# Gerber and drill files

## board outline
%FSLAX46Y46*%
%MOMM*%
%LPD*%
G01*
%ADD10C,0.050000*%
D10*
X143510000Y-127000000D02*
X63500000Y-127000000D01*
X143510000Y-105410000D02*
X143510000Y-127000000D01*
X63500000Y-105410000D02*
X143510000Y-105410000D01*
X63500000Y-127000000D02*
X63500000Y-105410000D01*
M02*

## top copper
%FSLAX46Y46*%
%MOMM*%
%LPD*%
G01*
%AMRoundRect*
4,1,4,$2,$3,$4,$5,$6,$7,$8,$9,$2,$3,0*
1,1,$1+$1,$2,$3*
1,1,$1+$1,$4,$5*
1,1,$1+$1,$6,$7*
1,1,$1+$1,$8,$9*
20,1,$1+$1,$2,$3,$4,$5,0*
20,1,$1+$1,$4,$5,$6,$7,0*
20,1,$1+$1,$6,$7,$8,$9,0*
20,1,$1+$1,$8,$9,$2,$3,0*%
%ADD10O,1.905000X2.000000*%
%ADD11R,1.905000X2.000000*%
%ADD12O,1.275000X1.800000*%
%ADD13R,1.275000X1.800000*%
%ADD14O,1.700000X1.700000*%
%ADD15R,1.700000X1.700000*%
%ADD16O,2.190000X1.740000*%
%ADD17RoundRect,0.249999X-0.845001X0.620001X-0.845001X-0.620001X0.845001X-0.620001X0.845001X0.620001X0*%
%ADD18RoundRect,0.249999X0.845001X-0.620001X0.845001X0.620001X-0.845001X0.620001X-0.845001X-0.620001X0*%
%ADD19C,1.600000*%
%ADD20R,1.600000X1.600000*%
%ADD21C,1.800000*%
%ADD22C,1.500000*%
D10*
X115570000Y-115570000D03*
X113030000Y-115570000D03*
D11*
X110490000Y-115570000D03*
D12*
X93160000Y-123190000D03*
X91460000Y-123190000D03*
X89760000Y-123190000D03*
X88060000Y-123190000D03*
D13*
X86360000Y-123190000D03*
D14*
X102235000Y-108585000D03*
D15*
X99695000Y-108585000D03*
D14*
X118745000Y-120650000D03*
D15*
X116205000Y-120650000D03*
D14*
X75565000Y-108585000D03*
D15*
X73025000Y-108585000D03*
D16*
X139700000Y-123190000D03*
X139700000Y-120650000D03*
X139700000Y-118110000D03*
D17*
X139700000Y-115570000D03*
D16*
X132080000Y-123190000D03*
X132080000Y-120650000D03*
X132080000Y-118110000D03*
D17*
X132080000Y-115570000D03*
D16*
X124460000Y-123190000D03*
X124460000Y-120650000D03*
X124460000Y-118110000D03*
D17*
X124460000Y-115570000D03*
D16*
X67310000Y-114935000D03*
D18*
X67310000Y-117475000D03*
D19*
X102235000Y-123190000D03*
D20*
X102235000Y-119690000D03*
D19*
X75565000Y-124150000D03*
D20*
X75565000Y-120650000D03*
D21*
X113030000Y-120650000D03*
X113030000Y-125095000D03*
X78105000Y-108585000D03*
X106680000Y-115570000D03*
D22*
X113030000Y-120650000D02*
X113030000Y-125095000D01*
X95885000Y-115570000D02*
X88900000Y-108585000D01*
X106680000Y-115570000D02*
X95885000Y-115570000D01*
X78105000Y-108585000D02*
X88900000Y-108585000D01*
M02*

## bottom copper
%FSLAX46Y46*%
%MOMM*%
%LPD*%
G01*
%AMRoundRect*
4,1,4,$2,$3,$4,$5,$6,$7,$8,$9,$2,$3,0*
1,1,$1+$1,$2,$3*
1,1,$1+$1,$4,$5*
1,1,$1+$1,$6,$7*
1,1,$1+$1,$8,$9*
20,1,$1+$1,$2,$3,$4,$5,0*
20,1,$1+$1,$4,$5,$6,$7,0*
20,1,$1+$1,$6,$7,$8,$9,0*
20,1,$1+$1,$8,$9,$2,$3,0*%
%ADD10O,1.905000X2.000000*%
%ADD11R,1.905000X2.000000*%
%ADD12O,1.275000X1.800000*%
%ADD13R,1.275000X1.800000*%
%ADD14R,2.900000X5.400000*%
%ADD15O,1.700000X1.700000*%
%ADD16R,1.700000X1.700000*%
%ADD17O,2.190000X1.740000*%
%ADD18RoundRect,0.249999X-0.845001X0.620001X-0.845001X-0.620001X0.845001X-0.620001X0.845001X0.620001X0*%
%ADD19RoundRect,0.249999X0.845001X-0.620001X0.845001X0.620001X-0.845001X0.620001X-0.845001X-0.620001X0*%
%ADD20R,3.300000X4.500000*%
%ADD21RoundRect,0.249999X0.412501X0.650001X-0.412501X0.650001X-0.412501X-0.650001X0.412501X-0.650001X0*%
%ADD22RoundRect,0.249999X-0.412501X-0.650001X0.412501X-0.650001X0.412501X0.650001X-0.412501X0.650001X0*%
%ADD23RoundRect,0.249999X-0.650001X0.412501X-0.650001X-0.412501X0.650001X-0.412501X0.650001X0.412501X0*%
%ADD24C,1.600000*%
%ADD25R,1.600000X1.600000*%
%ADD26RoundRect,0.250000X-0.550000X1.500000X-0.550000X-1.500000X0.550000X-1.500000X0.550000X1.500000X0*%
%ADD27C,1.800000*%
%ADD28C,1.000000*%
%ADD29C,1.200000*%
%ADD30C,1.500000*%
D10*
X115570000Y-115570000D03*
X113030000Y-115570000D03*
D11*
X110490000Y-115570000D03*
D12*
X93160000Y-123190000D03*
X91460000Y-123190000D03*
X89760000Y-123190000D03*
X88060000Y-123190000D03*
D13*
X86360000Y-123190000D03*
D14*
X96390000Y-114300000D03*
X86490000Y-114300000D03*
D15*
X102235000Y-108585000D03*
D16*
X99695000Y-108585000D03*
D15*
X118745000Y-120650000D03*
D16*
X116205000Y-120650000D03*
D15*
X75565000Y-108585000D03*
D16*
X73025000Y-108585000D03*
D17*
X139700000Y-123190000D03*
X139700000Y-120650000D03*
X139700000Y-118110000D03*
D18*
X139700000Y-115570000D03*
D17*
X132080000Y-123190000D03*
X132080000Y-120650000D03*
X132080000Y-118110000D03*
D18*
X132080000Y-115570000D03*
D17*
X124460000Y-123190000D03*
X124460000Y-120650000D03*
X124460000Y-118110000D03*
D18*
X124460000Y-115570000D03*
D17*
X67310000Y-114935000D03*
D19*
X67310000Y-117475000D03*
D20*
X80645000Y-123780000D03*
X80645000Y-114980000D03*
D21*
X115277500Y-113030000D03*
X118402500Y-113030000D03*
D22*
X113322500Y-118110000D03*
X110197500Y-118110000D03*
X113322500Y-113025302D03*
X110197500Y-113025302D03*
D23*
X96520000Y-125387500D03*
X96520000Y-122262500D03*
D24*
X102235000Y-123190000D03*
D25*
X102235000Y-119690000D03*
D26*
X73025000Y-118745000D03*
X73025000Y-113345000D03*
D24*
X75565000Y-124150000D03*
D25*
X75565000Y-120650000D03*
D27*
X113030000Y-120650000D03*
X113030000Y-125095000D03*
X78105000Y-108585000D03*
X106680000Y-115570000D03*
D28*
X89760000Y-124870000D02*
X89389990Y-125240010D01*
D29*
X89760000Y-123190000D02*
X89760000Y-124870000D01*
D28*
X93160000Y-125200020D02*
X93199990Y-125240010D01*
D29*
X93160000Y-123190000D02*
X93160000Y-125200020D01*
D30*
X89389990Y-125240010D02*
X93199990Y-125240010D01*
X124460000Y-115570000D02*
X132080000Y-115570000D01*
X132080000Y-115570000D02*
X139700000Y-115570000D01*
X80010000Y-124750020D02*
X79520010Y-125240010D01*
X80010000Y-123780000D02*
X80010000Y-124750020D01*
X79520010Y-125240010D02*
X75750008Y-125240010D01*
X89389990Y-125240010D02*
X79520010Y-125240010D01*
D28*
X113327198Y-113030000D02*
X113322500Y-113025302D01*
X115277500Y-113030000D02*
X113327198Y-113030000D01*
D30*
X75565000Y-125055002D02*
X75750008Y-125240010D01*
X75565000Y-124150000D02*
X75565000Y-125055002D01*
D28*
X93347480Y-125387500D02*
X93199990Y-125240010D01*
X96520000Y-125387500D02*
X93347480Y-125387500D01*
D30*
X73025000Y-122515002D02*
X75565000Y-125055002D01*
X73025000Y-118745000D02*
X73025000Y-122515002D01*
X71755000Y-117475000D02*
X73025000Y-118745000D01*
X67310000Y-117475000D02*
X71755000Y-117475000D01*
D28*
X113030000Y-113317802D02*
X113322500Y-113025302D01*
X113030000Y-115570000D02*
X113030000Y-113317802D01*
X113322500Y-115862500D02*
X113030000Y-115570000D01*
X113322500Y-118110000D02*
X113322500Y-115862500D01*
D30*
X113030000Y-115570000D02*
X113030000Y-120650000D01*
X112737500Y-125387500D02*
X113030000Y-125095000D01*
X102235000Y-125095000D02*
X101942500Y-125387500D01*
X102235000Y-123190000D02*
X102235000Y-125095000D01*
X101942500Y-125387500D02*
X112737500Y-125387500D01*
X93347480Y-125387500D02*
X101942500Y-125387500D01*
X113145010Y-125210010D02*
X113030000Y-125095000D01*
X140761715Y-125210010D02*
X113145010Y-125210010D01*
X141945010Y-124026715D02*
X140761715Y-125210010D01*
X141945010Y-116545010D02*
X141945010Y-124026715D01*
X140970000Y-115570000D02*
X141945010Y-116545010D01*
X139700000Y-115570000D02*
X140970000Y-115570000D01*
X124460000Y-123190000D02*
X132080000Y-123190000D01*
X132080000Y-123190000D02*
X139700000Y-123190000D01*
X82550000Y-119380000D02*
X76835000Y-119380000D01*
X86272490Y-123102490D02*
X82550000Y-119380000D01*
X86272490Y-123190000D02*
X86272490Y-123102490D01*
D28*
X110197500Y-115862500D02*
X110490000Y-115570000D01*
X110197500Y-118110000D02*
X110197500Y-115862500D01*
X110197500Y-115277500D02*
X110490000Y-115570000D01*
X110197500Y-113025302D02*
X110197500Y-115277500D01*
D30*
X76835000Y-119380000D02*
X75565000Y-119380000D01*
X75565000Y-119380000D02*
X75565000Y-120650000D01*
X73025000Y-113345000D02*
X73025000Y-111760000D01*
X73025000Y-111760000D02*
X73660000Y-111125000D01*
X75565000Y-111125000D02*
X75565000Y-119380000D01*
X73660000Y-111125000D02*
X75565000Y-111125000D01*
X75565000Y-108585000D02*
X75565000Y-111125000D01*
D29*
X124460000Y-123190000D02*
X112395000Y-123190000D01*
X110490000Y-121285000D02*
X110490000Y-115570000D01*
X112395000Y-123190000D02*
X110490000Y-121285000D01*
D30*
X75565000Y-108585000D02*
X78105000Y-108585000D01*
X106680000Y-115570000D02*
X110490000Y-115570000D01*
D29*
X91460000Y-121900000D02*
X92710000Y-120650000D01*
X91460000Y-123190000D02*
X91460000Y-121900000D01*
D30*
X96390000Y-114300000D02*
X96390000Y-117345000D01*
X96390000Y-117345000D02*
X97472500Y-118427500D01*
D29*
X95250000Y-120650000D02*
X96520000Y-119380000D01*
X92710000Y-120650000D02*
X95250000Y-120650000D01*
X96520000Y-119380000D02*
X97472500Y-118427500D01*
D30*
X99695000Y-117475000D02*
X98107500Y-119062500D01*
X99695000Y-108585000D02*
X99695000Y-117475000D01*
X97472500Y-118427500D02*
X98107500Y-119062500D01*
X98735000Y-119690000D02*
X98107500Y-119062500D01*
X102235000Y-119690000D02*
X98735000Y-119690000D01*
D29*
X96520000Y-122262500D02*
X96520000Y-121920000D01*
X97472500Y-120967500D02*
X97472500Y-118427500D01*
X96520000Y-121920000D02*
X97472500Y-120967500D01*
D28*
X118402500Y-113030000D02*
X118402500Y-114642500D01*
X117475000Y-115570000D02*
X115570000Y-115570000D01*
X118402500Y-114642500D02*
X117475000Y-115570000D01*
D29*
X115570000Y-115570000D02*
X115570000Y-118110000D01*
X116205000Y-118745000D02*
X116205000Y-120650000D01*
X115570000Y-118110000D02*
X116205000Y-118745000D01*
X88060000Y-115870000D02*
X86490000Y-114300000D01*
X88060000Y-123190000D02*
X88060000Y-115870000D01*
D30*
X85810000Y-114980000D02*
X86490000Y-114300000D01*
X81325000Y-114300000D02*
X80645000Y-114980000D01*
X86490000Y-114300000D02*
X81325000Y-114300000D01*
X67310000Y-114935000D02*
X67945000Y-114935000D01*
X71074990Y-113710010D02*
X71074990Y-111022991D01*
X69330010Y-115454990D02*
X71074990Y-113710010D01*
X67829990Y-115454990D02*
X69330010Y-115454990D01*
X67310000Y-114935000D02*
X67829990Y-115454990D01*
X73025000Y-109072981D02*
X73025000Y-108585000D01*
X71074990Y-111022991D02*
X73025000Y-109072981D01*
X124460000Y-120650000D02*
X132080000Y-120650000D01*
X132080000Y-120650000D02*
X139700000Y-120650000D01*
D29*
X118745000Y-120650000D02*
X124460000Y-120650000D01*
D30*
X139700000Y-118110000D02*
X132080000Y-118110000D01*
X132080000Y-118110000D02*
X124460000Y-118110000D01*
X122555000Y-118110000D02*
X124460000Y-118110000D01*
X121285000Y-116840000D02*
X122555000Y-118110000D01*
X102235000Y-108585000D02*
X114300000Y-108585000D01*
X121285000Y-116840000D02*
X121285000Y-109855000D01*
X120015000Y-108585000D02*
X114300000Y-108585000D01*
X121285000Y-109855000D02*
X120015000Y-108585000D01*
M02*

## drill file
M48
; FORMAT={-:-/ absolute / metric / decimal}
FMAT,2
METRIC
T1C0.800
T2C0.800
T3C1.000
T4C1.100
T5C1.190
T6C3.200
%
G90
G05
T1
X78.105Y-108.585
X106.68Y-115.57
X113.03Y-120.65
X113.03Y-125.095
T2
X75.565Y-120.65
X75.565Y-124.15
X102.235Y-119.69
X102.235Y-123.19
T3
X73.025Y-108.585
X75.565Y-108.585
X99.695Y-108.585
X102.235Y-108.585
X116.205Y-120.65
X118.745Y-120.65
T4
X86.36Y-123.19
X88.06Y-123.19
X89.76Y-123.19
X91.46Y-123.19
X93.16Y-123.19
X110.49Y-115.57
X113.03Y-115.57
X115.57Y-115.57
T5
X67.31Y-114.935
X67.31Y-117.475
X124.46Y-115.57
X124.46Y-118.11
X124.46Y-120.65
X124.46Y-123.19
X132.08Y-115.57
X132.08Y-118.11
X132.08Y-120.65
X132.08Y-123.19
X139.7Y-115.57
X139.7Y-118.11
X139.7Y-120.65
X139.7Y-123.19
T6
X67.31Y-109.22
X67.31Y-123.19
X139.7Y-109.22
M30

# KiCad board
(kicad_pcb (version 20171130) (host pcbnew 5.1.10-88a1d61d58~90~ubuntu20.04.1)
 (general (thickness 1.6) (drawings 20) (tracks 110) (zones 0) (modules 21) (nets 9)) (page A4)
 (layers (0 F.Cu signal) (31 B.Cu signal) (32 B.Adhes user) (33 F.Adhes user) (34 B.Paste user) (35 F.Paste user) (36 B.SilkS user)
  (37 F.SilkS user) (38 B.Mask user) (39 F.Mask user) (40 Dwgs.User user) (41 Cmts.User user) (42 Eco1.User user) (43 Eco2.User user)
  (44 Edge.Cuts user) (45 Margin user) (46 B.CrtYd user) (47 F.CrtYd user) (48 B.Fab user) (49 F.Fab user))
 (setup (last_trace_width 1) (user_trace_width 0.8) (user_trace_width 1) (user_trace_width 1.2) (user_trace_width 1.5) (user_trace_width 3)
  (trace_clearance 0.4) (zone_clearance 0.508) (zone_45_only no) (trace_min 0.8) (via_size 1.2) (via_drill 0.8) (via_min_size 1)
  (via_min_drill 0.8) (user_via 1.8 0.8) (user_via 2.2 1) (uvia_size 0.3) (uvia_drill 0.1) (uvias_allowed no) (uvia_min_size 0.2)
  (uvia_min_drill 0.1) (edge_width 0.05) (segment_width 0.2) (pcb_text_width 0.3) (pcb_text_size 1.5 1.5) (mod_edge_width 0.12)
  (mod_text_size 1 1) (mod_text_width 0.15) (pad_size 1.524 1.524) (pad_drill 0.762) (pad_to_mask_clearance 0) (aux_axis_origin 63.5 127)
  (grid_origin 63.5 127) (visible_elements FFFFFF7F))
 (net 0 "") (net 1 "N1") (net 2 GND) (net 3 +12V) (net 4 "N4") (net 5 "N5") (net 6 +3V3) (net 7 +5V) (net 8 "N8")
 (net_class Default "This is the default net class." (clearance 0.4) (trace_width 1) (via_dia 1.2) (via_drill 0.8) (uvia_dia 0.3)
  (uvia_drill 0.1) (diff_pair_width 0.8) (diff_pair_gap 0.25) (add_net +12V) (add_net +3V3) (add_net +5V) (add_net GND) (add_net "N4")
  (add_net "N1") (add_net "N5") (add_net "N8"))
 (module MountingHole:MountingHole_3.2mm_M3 (layer F.Cu) (at 139.7 109.22)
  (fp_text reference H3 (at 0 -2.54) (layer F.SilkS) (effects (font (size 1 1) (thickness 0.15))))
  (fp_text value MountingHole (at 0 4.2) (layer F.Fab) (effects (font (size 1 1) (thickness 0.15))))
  (pad 1 np_thru_hole circle (at 0 0) (size 3.2 3.2) (drill 3.2) (layers *.Cu *.Mask)))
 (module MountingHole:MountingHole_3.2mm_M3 (layer F.Cu) (at 67.31 123.19)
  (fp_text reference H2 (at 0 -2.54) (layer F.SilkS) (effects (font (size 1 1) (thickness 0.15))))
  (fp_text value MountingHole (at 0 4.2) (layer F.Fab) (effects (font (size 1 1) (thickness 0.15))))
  (pad 1 np_thru_hole circle (at 0 0) (size 3.2 3.2) (drill 3.2) (layers *.Cu *.Mask)))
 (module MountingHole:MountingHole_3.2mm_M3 (layer F.Cu) (at 67.31 109.22)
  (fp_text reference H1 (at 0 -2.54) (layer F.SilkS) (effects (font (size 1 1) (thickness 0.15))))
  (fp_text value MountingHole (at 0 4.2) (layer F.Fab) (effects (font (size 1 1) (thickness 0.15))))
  (pad 1 np_thru_hole circle (at 0 0) (size 3.2 3.2) (drill 3.2) (layers *.Cu *.Mask)))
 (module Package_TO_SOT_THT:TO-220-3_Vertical (layer F.Cu) (at 110.49 115.57)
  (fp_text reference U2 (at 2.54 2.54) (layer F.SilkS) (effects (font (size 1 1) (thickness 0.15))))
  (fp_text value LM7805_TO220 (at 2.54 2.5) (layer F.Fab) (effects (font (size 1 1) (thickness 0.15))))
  (pad 3 thru_hole oval (at 5.08 0) (size 1.905 2) (drill 1.1) (layers *.Cu *.Mask) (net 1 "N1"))
  (pad 2 thru_hole oval (at 2.54 0) (size 1.905 2) (drill 1.1) (layers *.Cu *.Mask) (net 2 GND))
  (pad 1 thru_hole rect (at 0 0) (size 1.905 2) (drill 1.1) (layers *.Cu *.Mask) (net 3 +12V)))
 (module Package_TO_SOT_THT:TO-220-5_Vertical (layer F.Cu) (at 86.36 123.19)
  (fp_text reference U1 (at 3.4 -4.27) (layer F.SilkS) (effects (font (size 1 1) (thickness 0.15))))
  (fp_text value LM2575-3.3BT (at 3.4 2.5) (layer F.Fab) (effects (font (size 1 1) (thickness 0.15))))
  (pad 5 thru_hole oval (at 6.8 0) (size 1.275 1.8) (drill 1.1) (layers *.Cu *.Mask) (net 2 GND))
  (pad 4 thru_hole oval (at 5.1 0) (size 1.275 1.8) (drill 1.1) (layers *.Cu *.Mask) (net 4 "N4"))
  (pad 3 thru_hole oval (at 3.4 0) (size 1.275 1.8) (drill 1.1) (layers *.Cu *.Mask) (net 2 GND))
  (pad 2 thru_hole oval (at 1.7 0) (size 1.275 1.8) (drill 1.1) (layers *.Cu *.Mask) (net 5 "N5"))
  (pad 1 thru_hole rect (at 0 0) (size 1.275 1.8) (drill 1.1) (layers *.Cu *.Mask) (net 3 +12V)))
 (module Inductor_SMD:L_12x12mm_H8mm (layer B.Cu) (at 91.44 114.3)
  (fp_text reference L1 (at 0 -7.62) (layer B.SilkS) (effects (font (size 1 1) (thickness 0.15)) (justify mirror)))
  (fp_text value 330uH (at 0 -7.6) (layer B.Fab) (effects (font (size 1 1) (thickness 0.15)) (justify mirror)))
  (pad 2 smd rect (at 4.95 0) (size 2.9 5.4) (layers B.Cu B.Paste B.Mask) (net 4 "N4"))
  (pad 1 smd rect (at -4.95 0) (size 2.9 5.4) (layers B.Cu B.Paste B.Mask) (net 5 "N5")))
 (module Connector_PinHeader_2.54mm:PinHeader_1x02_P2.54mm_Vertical (layer F.Cu) (at 99.695 108.585 90)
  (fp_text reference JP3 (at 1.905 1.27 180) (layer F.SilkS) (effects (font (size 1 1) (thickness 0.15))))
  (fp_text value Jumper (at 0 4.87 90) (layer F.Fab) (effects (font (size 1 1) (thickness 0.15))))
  (pad 2 thru_hole oval (at 0 2.54 90) (size 1.7 1.7) (drill 1) (layers *.Cu *.Mask) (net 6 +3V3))
  (pad 1 thru_hole rect (at 0 0 90) (size 1.7 1.7) (drill 1) (layers *.Cu *.Mask) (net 4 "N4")))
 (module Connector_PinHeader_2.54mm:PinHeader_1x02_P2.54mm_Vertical (layer F.Cu) (at 116.205 120.65 90)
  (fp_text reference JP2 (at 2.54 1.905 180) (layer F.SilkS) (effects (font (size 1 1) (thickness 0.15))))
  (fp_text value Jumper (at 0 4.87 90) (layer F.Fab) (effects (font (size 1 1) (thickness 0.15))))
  (pad 2 thru_hole oval (at 0 2.54 90) (size 1.7 1.7) (drill 1) (layers *.Cu *.Mask) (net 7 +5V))
  (pad 1 thru_hole rect (at 0 0 90) (size 1.7 1.7) (drill 1) (layers *.Cu *.Mask) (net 1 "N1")))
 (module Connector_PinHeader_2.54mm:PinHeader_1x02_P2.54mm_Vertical (layer F.Cu) (at 73.025 108.585 90)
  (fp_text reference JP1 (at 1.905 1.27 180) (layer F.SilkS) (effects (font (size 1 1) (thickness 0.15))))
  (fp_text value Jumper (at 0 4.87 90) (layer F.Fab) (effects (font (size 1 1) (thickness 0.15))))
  (pad 2 thru_hole oval (at 0 2.54 90) (size 1.7 1.7) (drill 1) (layers *.Cu *.Mask) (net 3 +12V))
  (pad 1 thru_hole rect (at 0 0 90) (size 1.7 1.7) (drill 1) (layers *.Cu *.Mask) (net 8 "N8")))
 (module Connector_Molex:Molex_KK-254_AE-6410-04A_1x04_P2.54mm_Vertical (layer F.Cu) (at 139.7 115.57 270)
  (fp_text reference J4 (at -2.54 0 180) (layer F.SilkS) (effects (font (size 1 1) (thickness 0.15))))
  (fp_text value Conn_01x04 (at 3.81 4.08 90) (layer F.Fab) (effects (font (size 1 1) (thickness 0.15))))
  (pad 4 thru_hole oval (at 7.62 0 270) (size 1.74 2.19) (drill 1.19) (layers *.Cu *.Mask) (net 3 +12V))
  (pad 3 thru_hole oval (at 5.08 0 270) (size 1.74 2.19) (drill 1.19) (layers *.Cu *.Mask) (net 7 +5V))
  (pad 2 thru_hole oval (at 2.54 0 270) (size 1.74 2.19) (drill 1.19) (layers *.Cu *.Mask) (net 6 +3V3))
  (pad 1 thru_hole roundrect (at 0 0 270) (size 1.74 2.19) (drill 1.19) (layers *.Cu *.Mask) (roundrect_rratio 0.1436775862068966)
   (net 2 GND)))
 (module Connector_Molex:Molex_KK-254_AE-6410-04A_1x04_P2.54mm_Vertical (layer F.Cu) (at 132.08 115.57 270)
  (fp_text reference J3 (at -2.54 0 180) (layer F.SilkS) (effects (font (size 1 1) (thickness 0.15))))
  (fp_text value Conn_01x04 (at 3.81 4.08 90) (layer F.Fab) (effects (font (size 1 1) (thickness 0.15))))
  (pad 4 thru_hole oval (at 7.62 0 270) (size 1.74 2.19) (drill 1.19) (layers *.Cu *.Mask) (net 3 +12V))
  (pad 3 thru_hole oval (at 5.08 0 270) (size 1.74 2.19) (drill 1.19) (layers *.Cu *.Mask) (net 7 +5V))
  (pad 2 thru_hole oval (at 2.54 0 270) (size 1.74 2.19) (drill 1.19) (layers *.Cu *.Mask) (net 6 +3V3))
  (pad 1 thru_hole roundrect (at 0 0 270) (size 1.74 2.19) (drill 1.19) (layers *.Cu *.Mask) (roundrect_rratio 0.1436775862068966)
   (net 2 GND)))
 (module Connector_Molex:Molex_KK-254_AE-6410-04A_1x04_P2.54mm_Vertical (layer F.Cu) (at 124.46 115.57 270)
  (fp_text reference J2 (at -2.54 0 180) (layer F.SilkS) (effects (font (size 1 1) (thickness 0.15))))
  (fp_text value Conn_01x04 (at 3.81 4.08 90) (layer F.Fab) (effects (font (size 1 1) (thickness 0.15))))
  (pad 4 thru_hole oval (at 7.62 0 270) (size 1.74 2.19) (drill 1.19) (layers *.Cu *.Mask) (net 3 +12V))
  (pad 3 thru_hole oval (at 5.08 0 270) (size 1.74 2.19) (drill 1.19) (layers *.Cu *.Mask) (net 7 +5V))
  (pad 2 thru_hole oval (at 2.54 0 270) (size 1.74 2.19) (drill 1.19) (layers *.Cu *.Mask) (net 6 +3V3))
  (pad 1 thru_hole roundrect (at 0 0 270) (size 1.74 2.19) (drill 1.19) (layers *.Cu *.Mask) (roundrect_rratio 0.1436775862068966)
   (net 2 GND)))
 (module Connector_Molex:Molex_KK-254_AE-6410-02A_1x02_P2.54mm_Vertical (layer F.Cu) (at 67.31 117.475 90)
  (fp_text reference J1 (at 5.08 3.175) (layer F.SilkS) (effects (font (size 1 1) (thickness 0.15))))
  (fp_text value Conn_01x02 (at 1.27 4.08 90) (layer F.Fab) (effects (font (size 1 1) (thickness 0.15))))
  (pad 2 thru_hole oval (at 2.54 0 90) (size 1.74 2.19) (drill 1.19) (layers *.Cu *.Mask) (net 8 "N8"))
  (pad 1 thru_hole roundrect (at 0 0 90) (size 1.74 2.19) (drill 1.19) (layers *.Cu *.Mask) (roundrect_rratio 0.1436775862068966)
   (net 2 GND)))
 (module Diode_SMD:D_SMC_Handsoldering (layer B.Cu) (at 80.645 119.38 270)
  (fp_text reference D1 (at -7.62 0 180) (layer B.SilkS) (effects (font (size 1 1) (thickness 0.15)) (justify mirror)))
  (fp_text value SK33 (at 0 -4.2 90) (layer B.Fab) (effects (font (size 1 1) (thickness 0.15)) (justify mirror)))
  (pad 2 smd rect (at 4.4 0 180) (size 3.3 4.5) (layers B.Cu B.Paste B.Mask) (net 2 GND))
  (pad 1 smd rect (at -4.4 0 180) (size 3.3 4.5) (layers B.Cu B.Paste B.Mask) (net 5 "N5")))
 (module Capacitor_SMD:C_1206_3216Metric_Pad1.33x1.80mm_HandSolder (layer B.Cu) (at 116.84 113.03 180)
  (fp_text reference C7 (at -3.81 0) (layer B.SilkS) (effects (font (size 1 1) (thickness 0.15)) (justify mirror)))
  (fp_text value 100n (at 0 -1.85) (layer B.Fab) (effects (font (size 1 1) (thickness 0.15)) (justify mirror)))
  (pad 2 smd roundrect (at 1.5625 0 180) (size 1.325 1.8) (layers B.Cu B.Paste B.Mask) (roundrect_rratio 0.1886784905660377) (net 2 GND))
  (pad 1 smd roundrect (at -1.5625 0 180) (size 1.325 1.8) (layers B.Cu B.Paste B.Mask) (roundrect_rratio 0.1886784905660377) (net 1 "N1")))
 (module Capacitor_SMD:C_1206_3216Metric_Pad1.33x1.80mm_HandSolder (layer B.Cu) (at 111.76 118.11)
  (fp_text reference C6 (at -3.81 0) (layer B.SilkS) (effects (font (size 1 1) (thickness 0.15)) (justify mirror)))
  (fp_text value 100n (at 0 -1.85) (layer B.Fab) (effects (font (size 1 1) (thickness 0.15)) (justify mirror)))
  (pad 2 smd roundrect (at 1.5625 0) (size 1.325 1.8) (layers B.Cu B.Paste B.Mask) (roundrect_rratio 0.1886784905660377) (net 2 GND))
  (pad 1 smd roundrect (at -1.5625 0) (size 1.325 1.8) (layers B.Cu B.Paste B.Mask) (roundrect_rratio 0.1886784905660377) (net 3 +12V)))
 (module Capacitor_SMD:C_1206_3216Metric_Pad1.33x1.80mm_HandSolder (layer B.Cu) (at 111.76 113.025302)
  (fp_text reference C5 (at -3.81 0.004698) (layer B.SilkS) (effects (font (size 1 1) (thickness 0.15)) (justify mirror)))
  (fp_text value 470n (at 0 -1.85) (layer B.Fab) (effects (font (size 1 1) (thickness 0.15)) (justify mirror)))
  (pad 2 smd roundrect (at 1.5625 0) (size 1.325 1.8) (layers B.Cu B.Paste B.Mask) (roundrect_rratio 0.1886784905660377) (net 2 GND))
  (pad 1 smd roundrect (at -1.5625 0) (size 1.325 1.8) (layers B.Cu B.Paste B.Mask) (roundrect_rratio 0.1886784905660377) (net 3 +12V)))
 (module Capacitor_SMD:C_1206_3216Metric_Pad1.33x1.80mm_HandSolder (layer B.Cu) (at 96.52 123.825 270)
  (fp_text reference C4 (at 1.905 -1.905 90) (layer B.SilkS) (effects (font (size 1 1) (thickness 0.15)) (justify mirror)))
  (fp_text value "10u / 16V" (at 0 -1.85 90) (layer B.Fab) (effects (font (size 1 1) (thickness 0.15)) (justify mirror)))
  (pad 2 smd roundrect (at 1.5625 0 270) (size 1.325 1.8) (layers B.Cu B.Paste B.Mask) (roundrect_rratio 0.1886784905660377) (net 2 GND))
  (pad 1 smd roundrect (at -1.5625 0 270) (size 1.325 1.8) (layers B.Cu B.Paste B.Mask) (roundrect_rratio 0.1886784905660377) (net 4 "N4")))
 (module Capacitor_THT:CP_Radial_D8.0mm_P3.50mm (layer F.Cu) (at 102.235 119.69 270)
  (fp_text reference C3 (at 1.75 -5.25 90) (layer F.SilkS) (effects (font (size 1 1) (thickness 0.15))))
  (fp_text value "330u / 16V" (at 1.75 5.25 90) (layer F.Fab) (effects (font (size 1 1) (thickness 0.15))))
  (pad 2 thru_hole circle (at 3.5 0 270) (size 1.6 1.6) (drill 0.8) (layers *.Cu *.Mask) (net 2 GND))
  (pad 1 thru_hole rect (at 0 0 270) (size 1.6 1.6) (drill 0.8) (layers *.Cu *.Mask) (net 4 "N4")))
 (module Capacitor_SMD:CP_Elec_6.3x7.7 (layer B.Cu) (at 73.025 116.045 270)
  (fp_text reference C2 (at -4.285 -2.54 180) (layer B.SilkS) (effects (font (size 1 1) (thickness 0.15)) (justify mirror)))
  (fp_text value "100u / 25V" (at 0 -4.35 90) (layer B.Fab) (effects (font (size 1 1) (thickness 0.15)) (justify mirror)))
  (pad 2 smd roundrect (at 2.7 0 270) (size 3.5 1.6) (layers B.Cu B.Paste B.Mask) (roundrect_rratio 0.15625) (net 2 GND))
  (pad 1 smd roundrect (at -2.7 0 270) (size 3.5 1.6) (layers B.Cu B.Paste B.Mask) (roundrect_rratio 0.15625) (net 3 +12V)))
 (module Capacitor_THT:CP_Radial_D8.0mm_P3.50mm (layer F.Cu) (at 75.565 120.65 270)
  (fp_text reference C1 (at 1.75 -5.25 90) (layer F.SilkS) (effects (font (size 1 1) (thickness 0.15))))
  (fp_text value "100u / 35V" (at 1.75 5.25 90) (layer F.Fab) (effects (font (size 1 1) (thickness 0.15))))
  (pad 2 thru_hole circle (at 3.5 0 270) (size 1.6 1.6) (drill 0.8) (layers *.Cu *.Mask) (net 2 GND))
  (pad 1 thru_hole rect (at 0 0 270) (size 1.6 1.6) (drill 0.8) (layers *.Cu *.Mask) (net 3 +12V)))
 (gr_line (start 143.51 127) (end 63.5 127) (layer Edge.Cuts) (width 0.05))
 (gr_line (start 143.51 105.41) (end 143.51 127) (layer Edge.Cuts) (width 0.05))
 (gr_line (start 63.5 105.41) (end 143.51 105.41) (layer Edge.Cuts) (width 0.05))
 (gr_line (start 63.5 127) (end 63.5 105.41) (layer Edge.Cuts) (width 0.05))
 (segment (start 89.76 124.87) (end 89.38999 125.24001) (width 1) (layer B.Cu) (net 2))
 (segment (start 89.76 123.19) (end 89.76 124.87) (width 1.2) (layer B.Cu) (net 2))
 (segment (start 93.16 125.20002) (end 93.19999 125.24001) (width 1) (layer B.Cu) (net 2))
 (segment (start 93.16 123.19) (end 93.16 125.20002) (width 1.2) (layer B.Cu) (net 2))
 (segment (start 89.38999 125.24001) (end 93.19999 125.24001) (width 1.5) (layer B.Cu) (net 2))
 (segment (start 124.46 115.57) (end 132.08 115.57) (width 1.5) (layer B.Cu) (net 2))
 (segment (start 132.08 115.57) (end 139.7 115.57) (width 1.5) (layer B.Cu) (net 2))
 (segment (start 80.01 124.75002) (end 79.52001 125.24001) (width 1.5) (layer B.Cu) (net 2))
 (segment (start 80.01 123.78) (end 80.01 124.75002) (width 1.5) (layer B.Cu) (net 2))
 (segment (start 79.52001 125.24001) (end 75.750008 125.24001) (width 1.5) (layer B.Cu) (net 2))
 (segment (start 89.38999 125.24001) (end 79.52001 125.24001) (width 1.5) (layer B.Cu) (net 2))
 (segment (start 113.327198 113.03) (end 113.3225 113.025302) (width 1) (layer B.Cu) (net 2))
 (segment (start 115.2775 113.03) (end 113.327198 113.03) (width 1) (layer B.Cu) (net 2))
 (segment (start 75.565 125.055002) (end 75.750008 125.24001) (width 1.5) (layer B.Cu) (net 2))
 (segment (start 75.565 124.15) (end 75.565 125.055002) (width 1.5) (layer B.Cu) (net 2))
 (segment (start 93.34748 125.3875) (end 93.19999 125.24001) (width 1) (layer B.Cu) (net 2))
 (segment (start 96.52 125.3875) (end 93.34748 125.3875) (width 1) (layer B.Cu) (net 2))
 (segment (start 73.025 122.515002) (end 75.565 125.055002) (width 1.5) (layer B.Cu) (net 2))
 (segment (start 73.025 118.745) (end 73.025 122.515002) (width 1.5) (layer B.Cu) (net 2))
 (segment (start 71.755 117.475) (end 73.025 118.745) (width 1.5) (layer B.Cu) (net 2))
 (segment (start 67.31 117.475) (end 71.755 117.475) (width 1.5) (layer B.Cu) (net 2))
 (segment (start 113.03 113.317802) (end 113.3225 113.025302) (width 1) (layer B.Cu) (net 2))
 (segment (start 113.03 115.57) (end 113.03 113.317802) (width 1) (layer B.Cu) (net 2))
 (segment (start 113.3225 115.8625) (end 113.03 115.57) (width 1) (layer B.Cu) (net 2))
 (segment (start 113.3225 118.11) (end 113.3225 115.8625) (width 1) (layer B.Cu) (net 2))
 (via (at 113.03 120.65) (size 1.8) (drill 0.8) (layers F.Cu B.Cu) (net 2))
 (segment (start 113.03 115.57) (end 113.03 120.65) (width 1.5) (layer B.Cu) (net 2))
 (via (at 113.03 125.095) (size 1.8) (drill 0.8) (layers F.Cu B.Cu) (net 2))
 (segment (start 113.03 120.65) (end 113.03 125.095) (width 1.5) (layer F.Cu) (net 2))
 (segment (start 112.7375 125.3875) (end 113.03 125.095) (width 1.5) (layer B.Cu) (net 2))
 (segment (start 102.235 125.095) (end 101.9425 125.3875) (width 1.5) (layer B.Cu) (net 2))
 (segment (start 102.235 123.19) (end 102.235 125.095) (width 1.5) (layer B.Cu) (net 2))
 (segment (start 101.9425 125.3875) (end 112.7375 125.3875) (width 1.5) (layer B.Cu) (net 2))
 (segment (start 93.34748 125.3875) (end 101.9425 125.3875) (width 1.5) (layer B.Cu) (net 2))
 (segment (start 113.14501 125.21001) (end 113.03 125.095) (width 1.5) (layer B.Cu) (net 2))
 (segment (start 140.761715 125.21001) (end 113.14501 125.21001) (width 1.5) (layer B.Cu) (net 2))
 (segment (start 141.94501 124.026715) (end 140.761715 125.21001) (width 1.5) (layer B.Cu) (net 2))
 (segment (start 141.94501 116.54501) (end 141.94501 124.026715) (width 1.5) (layer B.Cu) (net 2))
 (segment (start 140.97 115.57) (end 141.94501 116.54501) (width 1.5) (layer B.Cu) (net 2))
 (segment (start 139.7 115.57) (end 140.97 115.57) (width 1.5) (layer B.Cu) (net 2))
 (segment (start 124.46 123.19) (end 132.08 123.19) (width 1.5) (layer B.Cu) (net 3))
 (segment (start 132.08 123.19) (end 139.7 123.19) (width 1.5) (layer B.Cu) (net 3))
 (segment (start 82.55 119.38) (end 76.835 119.38) (width 1.5) (layer B.Cu) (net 3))
 (segment (start 86.27249 123.10249) (end 82.55 119.38) (width 1.5) (layer B.Cu) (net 3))
 (segment (start 86.27249 123.19) (end 86.27249 123.10249) (width 1.5) (layer B.Cu) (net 3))
 (segment (start 110.1975 115.8625) (end 110.49 115.57) (width 1) (layer B.Cu) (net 3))
 (segment (start 110.1975 118.11) (end 110.1975 115.8625) (width 1) (layer B.Cu) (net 3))
 (segment (start 110.1975 115.2775) (end 110.49 115.57) (width 1) (layer B.Cu) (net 3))
 (segment (start 110.1975 113.025302) (end 110.1975 115.2775) (width 1) (layer B.Cu) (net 3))
 (segment (start 76.835 119.38) (end 75.565 119.38) (width 1.5) (layer B.Cu) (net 3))
 (segment (start 75.565 119.38) (end 75.565 120.65) (width 1.5) (layer B.Cu) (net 3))
 (segment (start 73.025 113.345) (end 73.025 111.76) (width 1.5) (layer B.Cu) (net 3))
 (segment (start 73.025 111.76) (end 73.66 111.125) (width 1.5) (layer B.Cu) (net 3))
 (segment (start 75.565 111.125) (end 75.565 119.38) (width 1.5) (layer B.Cu) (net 3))
 (segment (start 73.66 111.125) (end 75.565 111.125) (width 1.5) (layer B.Cu) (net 3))
 (segment (start 75.565 108.585) (end 75.565 111.125) (width 1.5) (layer B.Cu) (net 3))
 (segment (start 124.46 123.19) (end 112.395 123.19) (width 1.2) (layer B.Cu) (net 3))
 (segment (start 110.49 121.285) (end 110.49 115.57) (width 1.2) (layer B.Cu) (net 3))
 (segment (start 112.395 123.19) (end 110.49 121.285) (width 1.2) (layer B.Cu) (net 3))
 (via (at 78.105 108.585) (size 1.8) (drill 0.8) (layers F.Cu B.Cu) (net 3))
 (segment (start 75.565 108.585) (end 78.105 108.585) (width 1.5) (layer B.Cu) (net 3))
 (via (at 106.68 115.57) (size 1.8) (drill 0.8) (layers F.Cu B.Cu) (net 3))
 (segment (start 106.68 115.57) (end 110.49 115.57) (width 1.5) (layer B.Cu) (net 3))
 (segment (start 95.885 115.57) (end 88.9 108.585) (width 1.5) (layer F.Cu) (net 3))
 (segment (start 106.68 115.57) (end 95.885 115.57) (width 1.5) (layer F.Cu) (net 3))
 (segment (start 78.105 108.585) (end 88.9 108.585) (width 1.5) (layer F.Cu) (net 3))
 (segment (start 91.46 121.9) (end 92.71 120.65) (width 1.2) (layer B.Cu) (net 4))
 (segment (start 91.46 123.19) (end 91.46 121.9) (width 1.2) (layer B.Cu) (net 4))
 (segment (start 96.39 114.3) (end 96.39 117.345) (width 1.5) (layer B.Cu) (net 4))
 (segment (start 96.39 117.345) (end 97.4725 118.4275) (width 1.5) (layer B.Cu) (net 4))
 (segment (start 95.25 120.65) (end 96.52 119.38) (width 1.2) (layer B.Cu) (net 4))
 (segment (start 92.71 120.65) (end 95.25 120.65) (width 1.2) (layer B.Cu) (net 4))
 (segment (start 96.52 119.38) (end 97.4725 118.4275) (width 1.2) (layer B.Cu) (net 4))
 (segment (start 99.695 117.475) (end 98.1075 119.0625) (width 1.5) (layer B.Cu) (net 4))
 (segment (start 99.695 108.585) (end 99.695 117.475) (width 1.5) (layer B.Cu) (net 4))
 (segment (start 97.4725 118.4275) (end 98.1075 119.0625) (width 1.5) (layer B.Cu) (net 4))
 (segment (start 98.735 119.69) (end 98.1075 119.0625) (width 1.5) (layer B.Cu) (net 4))
 (segment (start 102.235 119.69) (end 98.735 119.69) (width 1.5) (layer B.Cu) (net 4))
 (segment (start 96.52 122.2625) (end 96.52 121.92) (width 1.2) (layer B.Cu) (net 4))
 (segment (start 97.4725 120.9675) (end 97.4725 118.4275) (width 1.2) (layer B.Cu) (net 4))
 (segment (start 96.52 121.92) (end 97.4725 120.9675) (width 1.2) (layer B.Cu) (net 4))
 (segment (start 118.4025 113.03) (end 118.4025 114.6425) (width 1) (layer B.Cu) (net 1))
 (segment (start 117.475 115.57) (end 115.57 115.57) (width 1) (layer B.Cu) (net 1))
 (segment (start 118.4025 114.6425) (end 117.475 115.57) (width 1) (layer B.Cu) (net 1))
 (segment (start 115.57 115.57) (end 115.57 118.11) (width 1.2) (layer B.Cu) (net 1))
 (segment (start 116.205 118.745) (end 116.205 120.65) (width 1.2) (layer B.Cu) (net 1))
 (segment (start 115.57 118.11) (end 116.205 118.745) (width 1.2) (layer B.Cu) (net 1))
 (segment (start 88.06 115.87) (end 86.49 114.3) (width 1.2) (layer B.Cu) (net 5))
 (segment (start 88.06 123.19) (end 88.06 115.87) (width 1.2) (layer B.Cu) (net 5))
 (segment (start 85.81 114.98) (end 86.49 114.3) (width 1.5) (layer B.Cu) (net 5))
 (segment (start 81.325 114.3) (end 80.645 114.98) (width 1.5) (layer B.Cu) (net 5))
 (segment (start 86.49 114.3) (end 81.325 114.3) (width 1.5) (layer B.Cu) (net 5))
 (segment (start 67.31 114.935) (end 67.945 114.935) (width 1.5) (layer B.Cu) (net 8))
 (segment (start 71.07499 113.71001) (end 71.07499 111.022991) (width 1.5) (layer B.Cu) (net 8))
 (segment (start 69.33001 115.45499) (end 71.07499 113.71001) (width 1.5) (layer B.Cu) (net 8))
 (segment (start 67.82999 115.45499) (end 69.33001 115.45499) (width 1.5) (layer B.Cu) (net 8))
 (segment (start 67.31 114.935) (end 67.82999 115.45499) (width 1.5) (layer B.Cu) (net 8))
 (segment (start 73.025 109.072981) (end 73.025 108.585) (width 1.5) (layer B.Cu) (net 8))
 (segment (start 71.07499 111.022991) (end 73.025 109.072981) (width 1.5) (layer B.Cu) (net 8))
 (segment (start 124.46 120.65) (end 132.08 120.65) (width 1.5) (layer B.Cu) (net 7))
 (segment (start 132.08 120.65) (end 139.7 120.65) (width 1.5) (layer B.Cu) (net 7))
 (segment (start 118.745 120.65) (end 124.46 120.65) (width 1.2) (layer B.Cu) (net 7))
 (segment (start 139.7 118.11) (end 132.08 118.11) (width 1.5) (layer B.Cu) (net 6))
 (segment (start 132.08 118.11) (end 124.46 118.11) (width 1.5) (layer B.Cu) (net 6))
 (segment (start 122.555 118.11) (end 124.46 118.11) (width 1.5) (layer B.Cu) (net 6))
 (segment (start 121.285 116.84) (end 122.555 118.11) (width 1.5) (layer B.Cu) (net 6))
 (segment (start 102.235 108.585) (end 114.3 108.585) (width 1.5) (layer B.Cu) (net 6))
 (segment (start 121.285 116.84) (end 121.285 109.855) (width 1.5) (layer B.Cu) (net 6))
 (segment (start 120.015 108.585) (end 114.3 108.585) (width 1.5) (layer B.Cu) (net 6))
 (segment (start 121.285 109.855) (end 120.015 108.585) (width 1.5) (layer B.Cu) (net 6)))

